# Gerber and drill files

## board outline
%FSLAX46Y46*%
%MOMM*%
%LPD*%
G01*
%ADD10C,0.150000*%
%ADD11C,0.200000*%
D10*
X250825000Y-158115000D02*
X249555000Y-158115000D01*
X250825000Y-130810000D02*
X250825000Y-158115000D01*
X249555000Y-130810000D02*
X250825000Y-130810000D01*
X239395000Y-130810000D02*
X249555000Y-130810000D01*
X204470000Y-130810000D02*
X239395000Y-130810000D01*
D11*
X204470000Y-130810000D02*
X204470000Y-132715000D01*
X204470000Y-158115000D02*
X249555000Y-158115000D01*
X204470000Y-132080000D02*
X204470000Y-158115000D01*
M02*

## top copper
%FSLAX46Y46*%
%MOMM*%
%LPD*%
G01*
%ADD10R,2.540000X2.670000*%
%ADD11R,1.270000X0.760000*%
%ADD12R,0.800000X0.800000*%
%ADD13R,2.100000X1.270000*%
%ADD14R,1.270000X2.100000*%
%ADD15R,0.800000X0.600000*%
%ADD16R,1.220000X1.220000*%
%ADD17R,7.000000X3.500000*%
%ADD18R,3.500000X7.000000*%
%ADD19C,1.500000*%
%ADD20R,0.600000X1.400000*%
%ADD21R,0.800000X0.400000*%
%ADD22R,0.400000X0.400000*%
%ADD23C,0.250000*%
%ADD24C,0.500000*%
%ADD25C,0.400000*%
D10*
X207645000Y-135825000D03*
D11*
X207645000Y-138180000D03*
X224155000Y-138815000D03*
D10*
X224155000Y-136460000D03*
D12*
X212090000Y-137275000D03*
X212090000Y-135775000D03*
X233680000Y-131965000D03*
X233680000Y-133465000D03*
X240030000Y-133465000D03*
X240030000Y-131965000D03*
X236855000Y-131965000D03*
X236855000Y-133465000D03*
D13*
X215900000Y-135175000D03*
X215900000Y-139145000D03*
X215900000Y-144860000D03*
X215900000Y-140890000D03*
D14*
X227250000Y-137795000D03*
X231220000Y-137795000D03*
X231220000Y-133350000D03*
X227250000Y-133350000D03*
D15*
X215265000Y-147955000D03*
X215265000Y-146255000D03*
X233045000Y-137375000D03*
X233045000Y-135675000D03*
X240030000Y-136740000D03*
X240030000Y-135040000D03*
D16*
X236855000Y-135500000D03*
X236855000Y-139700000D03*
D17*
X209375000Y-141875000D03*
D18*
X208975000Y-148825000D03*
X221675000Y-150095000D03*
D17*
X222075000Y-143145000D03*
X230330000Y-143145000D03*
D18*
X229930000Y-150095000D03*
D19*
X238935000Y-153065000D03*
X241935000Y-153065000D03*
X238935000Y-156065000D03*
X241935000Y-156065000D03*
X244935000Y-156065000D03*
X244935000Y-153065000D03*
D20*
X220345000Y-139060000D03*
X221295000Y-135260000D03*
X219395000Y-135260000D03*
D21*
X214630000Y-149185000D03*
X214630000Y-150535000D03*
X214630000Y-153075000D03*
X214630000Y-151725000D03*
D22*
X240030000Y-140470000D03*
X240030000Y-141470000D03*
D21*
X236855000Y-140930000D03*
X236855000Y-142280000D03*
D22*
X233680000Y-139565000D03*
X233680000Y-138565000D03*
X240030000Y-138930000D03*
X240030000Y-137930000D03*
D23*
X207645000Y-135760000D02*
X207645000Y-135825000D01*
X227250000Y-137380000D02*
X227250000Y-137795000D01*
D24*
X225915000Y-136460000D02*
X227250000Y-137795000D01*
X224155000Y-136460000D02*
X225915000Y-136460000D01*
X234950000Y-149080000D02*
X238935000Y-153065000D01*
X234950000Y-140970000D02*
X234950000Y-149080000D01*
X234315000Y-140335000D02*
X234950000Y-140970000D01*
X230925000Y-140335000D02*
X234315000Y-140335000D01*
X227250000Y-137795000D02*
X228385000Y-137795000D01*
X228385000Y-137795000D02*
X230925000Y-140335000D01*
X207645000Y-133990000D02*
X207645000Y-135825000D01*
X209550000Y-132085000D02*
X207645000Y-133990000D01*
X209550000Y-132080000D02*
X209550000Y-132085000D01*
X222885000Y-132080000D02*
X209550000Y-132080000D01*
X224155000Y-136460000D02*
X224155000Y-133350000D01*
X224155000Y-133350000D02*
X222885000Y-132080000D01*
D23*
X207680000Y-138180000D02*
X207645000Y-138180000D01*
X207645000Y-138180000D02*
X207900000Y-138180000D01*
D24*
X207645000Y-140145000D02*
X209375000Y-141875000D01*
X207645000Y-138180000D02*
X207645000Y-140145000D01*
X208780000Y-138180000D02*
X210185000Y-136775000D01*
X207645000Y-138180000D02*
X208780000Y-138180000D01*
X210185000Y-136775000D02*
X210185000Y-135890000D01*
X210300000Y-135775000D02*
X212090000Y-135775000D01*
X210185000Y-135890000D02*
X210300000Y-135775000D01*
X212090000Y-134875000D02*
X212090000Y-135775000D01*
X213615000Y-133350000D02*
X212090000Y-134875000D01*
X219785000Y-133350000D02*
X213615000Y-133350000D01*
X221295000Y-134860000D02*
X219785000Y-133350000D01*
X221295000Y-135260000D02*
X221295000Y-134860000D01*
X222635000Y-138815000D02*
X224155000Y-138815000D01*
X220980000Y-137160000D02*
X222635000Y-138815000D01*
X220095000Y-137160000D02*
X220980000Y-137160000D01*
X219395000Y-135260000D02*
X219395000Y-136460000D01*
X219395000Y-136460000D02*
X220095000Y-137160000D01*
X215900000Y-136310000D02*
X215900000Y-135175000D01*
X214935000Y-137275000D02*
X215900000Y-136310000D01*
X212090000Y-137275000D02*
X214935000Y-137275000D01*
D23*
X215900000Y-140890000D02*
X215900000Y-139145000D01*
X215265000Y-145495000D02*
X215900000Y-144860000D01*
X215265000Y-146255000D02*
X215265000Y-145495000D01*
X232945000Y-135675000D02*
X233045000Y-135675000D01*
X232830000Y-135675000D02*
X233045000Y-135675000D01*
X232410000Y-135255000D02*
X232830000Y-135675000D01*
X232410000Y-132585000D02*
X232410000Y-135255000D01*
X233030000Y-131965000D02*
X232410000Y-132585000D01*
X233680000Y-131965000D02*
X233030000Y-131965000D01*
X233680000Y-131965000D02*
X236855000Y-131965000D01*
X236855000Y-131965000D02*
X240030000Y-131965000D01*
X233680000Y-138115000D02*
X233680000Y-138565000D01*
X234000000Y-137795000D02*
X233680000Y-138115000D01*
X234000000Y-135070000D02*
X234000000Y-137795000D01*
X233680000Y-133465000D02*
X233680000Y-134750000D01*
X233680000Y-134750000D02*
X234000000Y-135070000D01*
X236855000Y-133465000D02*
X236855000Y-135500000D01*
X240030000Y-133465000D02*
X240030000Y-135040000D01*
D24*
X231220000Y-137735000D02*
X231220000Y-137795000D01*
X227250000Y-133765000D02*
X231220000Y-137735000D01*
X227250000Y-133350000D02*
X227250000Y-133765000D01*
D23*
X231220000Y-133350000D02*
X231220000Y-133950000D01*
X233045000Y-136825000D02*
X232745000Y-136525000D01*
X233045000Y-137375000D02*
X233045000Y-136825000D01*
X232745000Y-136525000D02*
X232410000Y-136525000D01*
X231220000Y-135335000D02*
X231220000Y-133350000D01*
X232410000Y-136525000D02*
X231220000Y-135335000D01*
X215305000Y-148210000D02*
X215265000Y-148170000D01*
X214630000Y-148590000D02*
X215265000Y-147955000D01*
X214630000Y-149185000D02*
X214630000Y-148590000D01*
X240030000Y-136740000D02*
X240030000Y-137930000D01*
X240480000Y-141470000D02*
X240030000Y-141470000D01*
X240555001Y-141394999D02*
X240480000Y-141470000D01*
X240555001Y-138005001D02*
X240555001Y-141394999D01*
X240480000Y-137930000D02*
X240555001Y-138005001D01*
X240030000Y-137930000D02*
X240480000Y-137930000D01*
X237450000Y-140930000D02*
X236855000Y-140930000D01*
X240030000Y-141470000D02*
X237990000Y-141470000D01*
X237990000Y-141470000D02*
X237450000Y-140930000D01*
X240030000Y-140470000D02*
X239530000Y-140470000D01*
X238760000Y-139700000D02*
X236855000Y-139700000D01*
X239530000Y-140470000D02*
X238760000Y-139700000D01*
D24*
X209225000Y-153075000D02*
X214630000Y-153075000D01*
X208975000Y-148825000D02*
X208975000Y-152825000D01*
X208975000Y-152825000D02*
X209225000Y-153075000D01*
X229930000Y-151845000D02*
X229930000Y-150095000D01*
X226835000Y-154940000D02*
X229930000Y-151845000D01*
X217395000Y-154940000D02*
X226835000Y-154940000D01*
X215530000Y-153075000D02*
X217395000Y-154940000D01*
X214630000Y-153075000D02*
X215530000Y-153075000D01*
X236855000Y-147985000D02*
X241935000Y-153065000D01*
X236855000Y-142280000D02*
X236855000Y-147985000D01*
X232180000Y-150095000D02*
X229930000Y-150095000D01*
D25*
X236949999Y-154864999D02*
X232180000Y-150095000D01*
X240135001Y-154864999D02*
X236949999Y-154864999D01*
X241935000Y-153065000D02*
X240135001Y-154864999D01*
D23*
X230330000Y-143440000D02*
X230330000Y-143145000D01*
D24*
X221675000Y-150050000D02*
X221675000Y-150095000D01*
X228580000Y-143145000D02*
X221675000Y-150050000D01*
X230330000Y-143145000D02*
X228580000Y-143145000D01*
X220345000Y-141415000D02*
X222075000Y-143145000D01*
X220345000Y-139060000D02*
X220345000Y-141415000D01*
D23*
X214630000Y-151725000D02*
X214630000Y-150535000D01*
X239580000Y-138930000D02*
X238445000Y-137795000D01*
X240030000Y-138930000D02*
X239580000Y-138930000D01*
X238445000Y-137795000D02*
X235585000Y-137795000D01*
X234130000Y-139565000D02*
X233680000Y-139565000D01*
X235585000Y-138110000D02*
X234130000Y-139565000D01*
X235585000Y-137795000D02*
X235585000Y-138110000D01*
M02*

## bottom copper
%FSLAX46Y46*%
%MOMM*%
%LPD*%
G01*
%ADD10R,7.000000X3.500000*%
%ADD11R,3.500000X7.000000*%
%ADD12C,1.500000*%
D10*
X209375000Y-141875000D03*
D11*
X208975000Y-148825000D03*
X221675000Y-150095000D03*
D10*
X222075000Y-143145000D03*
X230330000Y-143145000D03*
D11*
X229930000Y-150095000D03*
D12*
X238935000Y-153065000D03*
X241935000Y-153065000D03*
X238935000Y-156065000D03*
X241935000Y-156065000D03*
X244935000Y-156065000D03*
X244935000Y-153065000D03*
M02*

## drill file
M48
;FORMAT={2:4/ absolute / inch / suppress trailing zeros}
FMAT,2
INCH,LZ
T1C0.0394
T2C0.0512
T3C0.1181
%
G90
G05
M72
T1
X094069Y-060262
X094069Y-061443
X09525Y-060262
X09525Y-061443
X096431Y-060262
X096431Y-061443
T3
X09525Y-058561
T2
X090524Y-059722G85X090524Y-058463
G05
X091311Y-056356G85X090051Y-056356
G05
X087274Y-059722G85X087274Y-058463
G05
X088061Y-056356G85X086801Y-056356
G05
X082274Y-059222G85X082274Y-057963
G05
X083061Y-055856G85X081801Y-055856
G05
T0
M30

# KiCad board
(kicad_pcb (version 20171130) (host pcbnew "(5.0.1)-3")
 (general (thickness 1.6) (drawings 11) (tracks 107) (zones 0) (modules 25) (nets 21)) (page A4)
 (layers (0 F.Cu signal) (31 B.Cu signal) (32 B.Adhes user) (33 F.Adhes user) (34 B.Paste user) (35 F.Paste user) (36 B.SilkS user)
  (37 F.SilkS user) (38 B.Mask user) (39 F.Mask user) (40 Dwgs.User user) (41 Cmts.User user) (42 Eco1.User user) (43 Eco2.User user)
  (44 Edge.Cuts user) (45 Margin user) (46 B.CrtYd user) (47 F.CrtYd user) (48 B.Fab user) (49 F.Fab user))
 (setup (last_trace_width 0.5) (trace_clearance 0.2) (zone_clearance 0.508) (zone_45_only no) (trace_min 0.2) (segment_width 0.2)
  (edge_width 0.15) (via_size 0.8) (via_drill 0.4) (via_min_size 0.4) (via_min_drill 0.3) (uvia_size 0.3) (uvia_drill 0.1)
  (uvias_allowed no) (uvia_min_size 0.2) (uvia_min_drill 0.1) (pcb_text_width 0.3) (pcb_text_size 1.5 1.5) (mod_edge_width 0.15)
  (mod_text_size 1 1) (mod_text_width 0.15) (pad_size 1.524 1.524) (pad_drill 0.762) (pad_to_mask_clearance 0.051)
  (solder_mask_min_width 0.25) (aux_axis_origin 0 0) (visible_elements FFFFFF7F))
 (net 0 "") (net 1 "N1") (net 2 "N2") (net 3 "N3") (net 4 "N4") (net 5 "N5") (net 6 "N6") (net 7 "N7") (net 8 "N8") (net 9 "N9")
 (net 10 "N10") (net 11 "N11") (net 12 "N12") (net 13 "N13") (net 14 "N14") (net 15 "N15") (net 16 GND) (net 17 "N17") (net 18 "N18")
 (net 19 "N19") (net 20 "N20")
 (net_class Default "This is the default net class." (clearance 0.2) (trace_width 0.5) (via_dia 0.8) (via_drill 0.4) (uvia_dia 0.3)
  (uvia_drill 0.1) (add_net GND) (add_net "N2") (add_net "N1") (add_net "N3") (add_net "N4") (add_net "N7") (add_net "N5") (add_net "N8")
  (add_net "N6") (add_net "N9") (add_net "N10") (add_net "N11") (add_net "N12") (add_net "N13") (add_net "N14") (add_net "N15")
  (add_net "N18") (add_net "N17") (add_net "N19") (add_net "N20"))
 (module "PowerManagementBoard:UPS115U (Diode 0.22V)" (layer F.Cu) (at 207.645 137.16 270)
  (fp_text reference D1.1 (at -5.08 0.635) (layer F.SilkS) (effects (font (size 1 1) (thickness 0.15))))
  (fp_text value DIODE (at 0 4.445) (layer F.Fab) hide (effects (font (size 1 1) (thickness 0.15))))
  (pad 2 smd rect (at -1.335 0 270) (size 2.67 2.54) (layers F.Cu F.Paste F.Mask) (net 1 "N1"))
  (pad 1 smd rect (at 1.02 0 270) (size 0.76 1.27) (layers F.Cu F.Paste F.Mask) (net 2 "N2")))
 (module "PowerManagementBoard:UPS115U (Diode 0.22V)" (layer F.Cu) (at 224.155 137.795 270)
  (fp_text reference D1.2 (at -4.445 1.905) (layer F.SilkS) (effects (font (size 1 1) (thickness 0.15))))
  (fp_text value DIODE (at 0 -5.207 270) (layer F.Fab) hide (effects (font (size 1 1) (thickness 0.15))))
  (pad 1 smd rect (at 1.02 0 270) (size 0.76 1.27) (layers F.Cu F.Paste F.Mask) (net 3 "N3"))
  (pad 2 smd rect (at -1.335 0 270) (size 2.67 2.54) (layers F.Cu F.Paste F.Mask) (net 1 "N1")))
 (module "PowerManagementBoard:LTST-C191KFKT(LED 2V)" (layer F.Cu) (at 212.09 136.525 90)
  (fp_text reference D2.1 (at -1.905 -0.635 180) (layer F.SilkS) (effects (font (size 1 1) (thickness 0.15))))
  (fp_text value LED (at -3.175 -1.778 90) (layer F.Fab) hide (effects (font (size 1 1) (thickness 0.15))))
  (pad 1 smd rect (at -0.75 0 90) (size 0.8 0.8) (layers F.Cu B.Adhes F.Paste F.Mask) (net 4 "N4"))
  (pad 2 smd rect (at 0.75 0 90) (size 0.8 0.8) (layers F.Cu F.Paste F.Mask) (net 2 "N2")))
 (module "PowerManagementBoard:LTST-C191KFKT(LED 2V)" (layer F.Cu) (at 233.68 132.715 90)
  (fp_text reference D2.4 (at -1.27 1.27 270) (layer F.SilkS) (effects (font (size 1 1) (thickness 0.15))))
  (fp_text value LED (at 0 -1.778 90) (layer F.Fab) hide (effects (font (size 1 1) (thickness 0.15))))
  (pad 2 smd rect (at 0.75 0 90) (size 0.8 0.8) (layers F.Cu F.Paste F.Mask) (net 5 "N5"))
  (pad 1 smd rect (at -0.75 0 90) (size 0.8 0.8) (layers F.Cu B.Adhes F.Paste F.Mask) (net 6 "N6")))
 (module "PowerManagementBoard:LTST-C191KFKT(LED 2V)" (layer F.Cu) (at 240.03 132.715 90)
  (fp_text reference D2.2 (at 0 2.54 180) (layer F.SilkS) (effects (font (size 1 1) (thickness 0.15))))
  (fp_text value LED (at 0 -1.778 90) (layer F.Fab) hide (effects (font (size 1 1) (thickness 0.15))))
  (pad 1 smd rect (at -0.75 0 90) (size 0.8 0.8) (layers F.Cu B.Adhes F.Paste F.Mask) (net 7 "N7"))
  (pad 2 smd rect (at 0.75 0 90) (size 0.8 0.8) (layers F.Cu F.Paste F.Mask) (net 5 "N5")))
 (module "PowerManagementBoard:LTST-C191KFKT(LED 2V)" (layer F.Cu) (at 236.855 132.715 90)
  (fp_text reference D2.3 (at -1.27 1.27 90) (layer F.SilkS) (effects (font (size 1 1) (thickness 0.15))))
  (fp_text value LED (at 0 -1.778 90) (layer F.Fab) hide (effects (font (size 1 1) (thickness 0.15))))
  (pad 2 smd rect (at 0.75 0 90) (size 0.8 0.8) (layers F.Cu F.Paste F.Mask) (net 5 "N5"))
  (pad 1 smd rect (at -0.75 0 90) (size 0.8 0.8) (layers F.Cu B.Adhes F.Paste F.Mask) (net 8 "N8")))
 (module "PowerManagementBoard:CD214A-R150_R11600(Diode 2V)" (layer F.Cu) (at 215.9 137.16 270)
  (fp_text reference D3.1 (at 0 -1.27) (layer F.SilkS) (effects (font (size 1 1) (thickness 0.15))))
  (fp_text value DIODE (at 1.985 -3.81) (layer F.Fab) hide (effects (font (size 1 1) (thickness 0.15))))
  (pad 1 smd rect (at -1.985 0 270) (size 1.27 2.1) (layers F.Cu B.Adhes F.Paste F.Mask) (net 4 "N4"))
  (pad 2 smd rect (at 1.985 0 270) (size 1.27 2.1) (layers F.Cu B.Adhes F.Paste F.Mask) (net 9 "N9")))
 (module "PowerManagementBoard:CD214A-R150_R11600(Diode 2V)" (layer F.Cu) (at 215.9 142.875 270)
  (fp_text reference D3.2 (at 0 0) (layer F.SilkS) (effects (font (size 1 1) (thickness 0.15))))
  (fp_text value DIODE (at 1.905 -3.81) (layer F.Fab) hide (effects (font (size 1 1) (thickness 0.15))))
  (pad 2 smd rect (at 1.985 0 270) (size 1.27 2.1) (layers F.Cu B.Adhes F.Paste F.Mask) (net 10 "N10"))
  (pad 1 smd rect (at -1.985 0 270) (size 1.27 2.1) (layers F.Cu B.Adhes F.Paste F.Mask) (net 9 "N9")))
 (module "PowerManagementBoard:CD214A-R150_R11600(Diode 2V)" (layer F.Cu) (at 229.235 137.795)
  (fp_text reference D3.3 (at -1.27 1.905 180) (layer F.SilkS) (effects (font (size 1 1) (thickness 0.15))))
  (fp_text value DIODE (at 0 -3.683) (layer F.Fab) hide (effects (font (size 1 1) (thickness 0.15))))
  (pad 1 smd rect (at -1.985 0) (size 1.27 2.1) (layers F.Cu B.Adhes F.Paste F.Mask) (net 1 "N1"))
  (pad 2 smd rect (at 1.985 0) (size 1.27 2.1) (layers F.Cu B.Adhes F.Paste F.Mask) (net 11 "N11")))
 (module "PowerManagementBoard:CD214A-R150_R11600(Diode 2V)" (layer F.Cu) (at 229.235 133.35)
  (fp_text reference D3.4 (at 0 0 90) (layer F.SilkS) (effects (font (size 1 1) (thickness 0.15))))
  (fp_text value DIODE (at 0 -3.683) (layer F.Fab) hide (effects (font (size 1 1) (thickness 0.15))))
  (pad 2 smd rect (at 1.985 0) (size 1.27 2.1) (layers F.Cu B.Adhes F.Paste F.Mask) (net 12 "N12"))
  (pad 1 smd rect (at -1.985 0) (size 1.27 2.1) (layers F.Cu B.Adhes F.Paste F.Mask) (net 11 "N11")))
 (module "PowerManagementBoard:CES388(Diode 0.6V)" (layer F.Cu) (at 215.265 147.105 270)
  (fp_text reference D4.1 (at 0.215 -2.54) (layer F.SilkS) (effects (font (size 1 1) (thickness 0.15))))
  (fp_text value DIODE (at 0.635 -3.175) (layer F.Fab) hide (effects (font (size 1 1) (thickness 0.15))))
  (pad 2 smd rect (at 0.85 0 270) (size 0.6 0.8) (layers F.Cu B.Adhes F.Paste F.Mask) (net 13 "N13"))
  (pad 1 smd rect (at -0.85 0 270) (size 0.6 0.8) (layers F.Cu B.Adhes F.Paste F.Mask) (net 10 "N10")))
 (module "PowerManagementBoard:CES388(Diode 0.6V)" (layer F.Cu) (at 233.045 136.525 90)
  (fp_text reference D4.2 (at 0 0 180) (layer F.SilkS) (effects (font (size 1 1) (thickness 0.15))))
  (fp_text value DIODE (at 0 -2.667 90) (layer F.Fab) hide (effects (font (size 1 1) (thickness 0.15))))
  (pad 1 smd rect (at -0.85 0 90) (size 0.6 0.8) (layers F.Cu B.Adhes F.Paste F.Mask) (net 12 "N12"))
  (pad 2 smd rect (at 0.85 0 90) (size 0.6 0.8) (layers F.Cu B.Adhes F.Paste F.Mask) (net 5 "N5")))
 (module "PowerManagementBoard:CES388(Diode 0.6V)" (layer F.Cu) (at 240.03 135.89 270)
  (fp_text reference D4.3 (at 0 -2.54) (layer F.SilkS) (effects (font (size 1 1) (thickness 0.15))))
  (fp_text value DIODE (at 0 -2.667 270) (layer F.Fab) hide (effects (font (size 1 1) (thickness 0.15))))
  (pad 2 smd rect (at 0.85 0 270) (size 0.6 0.8) (layers F.Cu B.Adhes F.Paste F.Mask) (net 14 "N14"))
  (pad 1 smd rect (at -0.85 0 270) (size 0.6 0.8) (layers F.Cu B.Adhes F.Paste F.Mask) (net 7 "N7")))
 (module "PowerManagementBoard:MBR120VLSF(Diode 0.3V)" (layer F.Cu) (at 236.855 137.6 90)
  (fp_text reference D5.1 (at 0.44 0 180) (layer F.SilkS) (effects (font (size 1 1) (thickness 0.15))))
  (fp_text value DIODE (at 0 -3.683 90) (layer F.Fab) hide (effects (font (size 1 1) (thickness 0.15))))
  (pad 1 smd rect (at 2.1 0 90) (size 1.22 1.22) (layers F.Cu B.Adhes F.Paste F.Mask) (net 8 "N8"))
  (pad 2 smd rect (at -2.1 0 90) (size 1.22 1.22) (layers F.Cu B.Adhes F.Paste F.Mask) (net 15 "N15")))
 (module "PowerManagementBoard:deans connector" (layer F.Cu) (at 206.375 142.875 180)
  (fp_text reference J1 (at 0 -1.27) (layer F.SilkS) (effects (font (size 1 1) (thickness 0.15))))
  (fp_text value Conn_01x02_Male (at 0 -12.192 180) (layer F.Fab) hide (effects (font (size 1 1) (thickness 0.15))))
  (pad 1 thru_hole rect (at -3 1 180) (size 7 3.5) (drill oval 4.5 1.3) (layers *.Cu *.Mask) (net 2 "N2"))
  (pad 2 thru_hole rect (at -2.6 -5.95 180) (size 3.5 7) (drill oval 1.3 4.5) (layers *.Cu *.Mask) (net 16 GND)))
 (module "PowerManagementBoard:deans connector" (layer F.Cu) (at 219.075 144.145 180)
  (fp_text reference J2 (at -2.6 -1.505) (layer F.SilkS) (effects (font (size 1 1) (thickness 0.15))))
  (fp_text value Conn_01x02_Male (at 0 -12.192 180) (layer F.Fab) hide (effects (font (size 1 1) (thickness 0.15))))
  (pad 2 thru_hole rect (at -2.6 -5.95 180) (size 3.5 7) (drill oval 1.3 4.5) (layers *.Cu *.Mask) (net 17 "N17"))
  (pad 1 thru_hole rect (at -3 1 180) (size 7 3.5) (drill oval 4.5 1.3) (layers *.Cu *.Mask) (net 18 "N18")))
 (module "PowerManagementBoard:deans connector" (layer F.Cu) (at 227.33 144.145 180)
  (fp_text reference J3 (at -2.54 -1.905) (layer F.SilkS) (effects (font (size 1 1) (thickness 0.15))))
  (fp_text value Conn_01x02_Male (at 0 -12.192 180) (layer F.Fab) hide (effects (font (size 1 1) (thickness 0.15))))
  (pad 1 thru_hole rect (at -3 1 180) (size 7 3.5) (drill oval 4.5 1.3) (layers *.Cu *.Mask) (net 17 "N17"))
  (pad 2 thru_hole rect (at -2.6 -5.95 180) (size 3.5 7) (drill oval 1.3 4.5) (layers *.Cu *.Mask) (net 16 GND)))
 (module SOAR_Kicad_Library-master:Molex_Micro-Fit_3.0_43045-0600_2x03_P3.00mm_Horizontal (layer F.Cu) (at 241.935 144.145 180)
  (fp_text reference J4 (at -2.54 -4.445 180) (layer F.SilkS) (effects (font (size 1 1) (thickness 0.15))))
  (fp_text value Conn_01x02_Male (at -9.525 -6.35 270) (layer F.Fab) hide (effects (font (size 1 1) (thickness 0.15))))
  (pad "" np_thru_hole circle (at 0 -4.6) (size 3 3) (drill 3) (layers *.Cu *.Mask))
  (pad 1 thru_hole circle (at 3 -8.92) (size 1.5 1.5) (drill 1) (layers *.Cu *.Mask) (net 1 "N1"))
  (pad 2 thru_hole circle (at 0 -8.92) (size 1.5 1.5) (drill 1) (layers *.Cu *.Mask) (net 16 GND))
  (pad 4 thru_hole circle (at 3 -11.92) (size 1.5 1.5) (drill 1) (layers *.Cu *.Mask))
  (pad 5 thru_hole circle (at 0 -11.92) (size 1.5 1.5) (drill 1) (layers *.Cu *.Mask))
  (pad 6 thru_hole circle (at -3 -11.92) (size 1.5 1.5) (drill 1) (layers *.Cu *.Mask))
  (pad 3 thru_hole circle (at -3 -8.92) (size 1.5 1.5) (drill 1) (layers *.Cu *.Mask)))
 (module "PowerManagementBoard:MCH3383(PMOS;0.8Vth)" (layer F.Cu) (at 220.345 137.16 180)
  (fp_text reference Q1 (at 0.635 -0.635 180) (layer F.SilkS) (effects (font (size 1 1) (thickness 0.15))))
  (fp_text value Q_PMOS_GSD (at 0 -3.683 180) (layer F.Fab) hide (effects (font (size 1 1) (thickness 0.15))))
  (pad 3 smd rect (at 0 -1.9 180) (size 0.6 1.4) (layers F.Cu F.Paste F.Mask) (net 18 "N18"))
  (pad 1 smd rect (at -0.95 1.9 180) (size 0.6 1.4) (layers F.Cu F.Paste F.Mask) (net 2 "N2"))
  (pad 2 smd rect (at 0.95 1.9 180) (size 0.6 1.4) (layers F.Cu F.Paste F.Mask) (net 3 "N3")))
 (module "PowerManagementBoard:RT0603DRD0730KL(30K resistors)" (layer F.Cu) (at 214.63 149.86 90)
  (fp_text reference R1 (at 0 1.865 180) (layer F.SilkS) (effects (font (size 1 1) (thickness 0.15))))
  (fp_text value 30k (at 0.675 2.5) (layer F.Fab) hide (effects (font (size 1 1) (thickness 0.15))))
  (pad 1 smd rect (at 0.675 0 90) (size 0.4 0.8) (layers F.Cu B.Adhes F.Paste F.Mask) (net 13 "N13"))
  (pad 2 smd rect (at -0.675 0 90) (size 0.4 0.8) (layers F.Cu B.Adhes F.Paste F.Mask) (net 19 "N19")))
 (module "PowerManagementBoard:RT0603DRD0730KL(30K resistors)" (layer F.Cu) (at 214.63 152.4 90)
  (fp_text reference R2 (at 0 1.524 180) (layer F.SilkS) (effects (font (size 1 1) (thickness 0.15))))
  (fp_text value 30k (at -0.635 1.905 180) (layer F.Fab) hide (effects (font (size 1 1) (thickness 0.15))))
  (pad 2 smd rect (at -0.675 0 90) (size 0.4 0.8) (layers F.Cu B.Adhes F.Paste F.Mask) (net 16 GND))
  (pad 1 smd rect (at 0.675 0 90) (size 0.4 0.8) (layers F.Cu B.Adhes F.Paste F.Mask) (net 19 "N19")))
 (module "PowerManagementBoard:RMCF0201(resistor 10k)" (layer F.Cu) (at 240.03 140.97 90)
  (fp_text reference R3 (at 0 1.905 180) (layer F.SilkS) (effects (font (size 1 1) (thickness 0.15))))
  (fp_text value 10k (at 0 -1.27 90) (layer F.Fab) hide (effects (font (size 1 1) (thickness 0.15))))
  (pad 1 smd rect (at 0.5 0 90) (size 0.4 0.4) (layers F.Cu B.Adhes F.Paste F.Mask) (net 15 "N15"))
  (pad 2 smd rect (at -0.5 0 90) (size 0.4 0.4) (layers F.Cu B.Adhes F.Paste F.Mask) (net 14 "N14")))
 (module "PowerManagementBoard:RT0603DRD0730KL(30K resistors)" (layer F.Cu) (at 236.855 141.605 90)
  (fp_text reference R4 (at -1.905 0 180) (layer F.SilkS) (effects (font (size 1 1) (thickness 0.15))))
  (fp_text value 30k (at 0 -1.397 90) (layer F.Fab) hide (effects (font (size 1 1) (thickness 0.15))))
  (pad 1 smd rect (at 0.675 0 90) (size 0.4 0.8) (layers F.Cu B.Adhes F.Paste F.Mask) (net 14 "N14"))
  (pad 2 smd rect (at -0.675 0 90) (size 0.4 0.8) (layers F.Cu B.Adhes F.Paste F.Mask) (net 16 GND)))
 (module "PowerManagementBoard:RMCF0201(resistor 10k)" (layer F.Cu) (at 233.68 139.065 90)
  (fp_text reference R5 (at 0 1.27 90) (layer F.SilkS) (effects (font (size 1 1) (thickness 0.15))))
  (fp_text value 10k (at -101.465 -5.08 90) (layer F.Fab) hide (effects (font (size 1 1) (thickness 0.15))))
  (pad 2 smd rect (at -0.5 0 90) (size 0.4 0.4) (layers F.Cu B.Adhes F.Paste F.Mask) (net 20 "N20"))
  (pad 1 smd rect (at 0.5 0 90) (size 0.4 0.4) (layers F.Cu B.Adhes F.Paste F.Mask) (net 6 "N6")))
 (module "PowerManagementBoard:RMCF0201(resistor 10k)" (layer F.Cu) (at 240.03 138.43 270)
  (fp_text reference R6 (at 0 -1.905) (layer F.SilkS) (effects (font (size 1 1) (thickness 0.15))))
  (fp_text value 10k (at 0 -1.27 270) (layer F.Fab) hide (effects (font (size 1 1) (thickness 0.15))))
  (pad 1 smd rect (at 0.5 0 270) (size 0.4 0.4) (layers F.Cu B.Adhes F.Paste F.Mask) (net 20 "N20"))
  (pad 2 smd rect (at -0.5 0 270) (size 0.4 0.4) (layers F.Cu B.Adhes F.Paste F.Mask) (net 14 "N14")))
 (gr_line (start 250.825 158.115) (end 249.555 158.115) (layer Edge.Cuts) (width 0.15))
 (gr_line (start 250.825 130.81) (end 250.825 158.115) (layer Edge.Cuts) (width 0.15))
 (gr_line (start 249.555 130.81) (end 250.825 130.81) (layer Edge.Cuts) (width 0.15))
 (gr_line (start 239.395 130.81) (end 249.555 130.81) (layer Edge.Cuts) (width 0.15))
 (gr_line (start 204.47 130.81) (end 239.395 130.81) (layer Edge.Cuts) (width 0.15))
 (gr_line (start 204.47 130.81) (end 204.47 132.715) (layer Edge.Cuts) (width 0.2))
 (gr_line (start 204.47 158.115) (end 249.555 158.115) (layer Edge.Cuts) (width 0.2))
 (gr_line (start 204.47 132.08) (end 204.47 158.115) (layer Edge.Cuts) (width 0.2))
 (segment (start 207.645 135.76) (end 207.645 135.825) (width 0.25) (layer F.Cu) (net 1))
 (segment (start 227.25 137.38) (end 227.25 137.795) (width 0.25) (layer F.Cu) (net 1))
 (segment (start 225.915 136.46) (end 227.25 137.795) (width 0.5) (layer F.Cu) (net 1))
 (segment (start 224.155 136.46) (end 225.915 136.46) (width 0.5) (layer F.Cu) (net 1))
 (segment (start 234.95 149.08) (end 238.935 153.065) (width 0.5) (layer F.Cu) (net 1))
 (segment (start 234.95 140.97) (end 234.95 149.08) (width 0.5) (layer F.Cu) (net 1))
 (segment (start 234.315 140.335) (end 234.95 140.97) (width 0.5) (layer F.Cu) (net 1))
 (segment (start 230.925 140.335) (end 234.315 140.335) (width 0.5) (layer F.Cu) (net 1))
 (segment (start 227.25 137.795) (end 228.385 137.795) (width 0.5) (layer F.Cu) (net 1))
 (segment (start 228.385 137.795) (end 230.925 140.335) (width 0.5) (layer F.Cu) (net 1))
 (segment (start 207.645 133.99) (end 207.645 135.825) (width 0.5) (layer F.Cu) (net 1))
 (segment (start 209.55 132.085) (end 207.645 133.99) (width 0.5) (layer F.Cu) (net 1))
 (segment (start 209.55 132.08) (end 209.55 132.085) (width 0.5) (layer F.Cu) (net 1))
 (segment (start 222.885 132.08) (end 209.55 132.08) (width 0.5) (layer F.Cu) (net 1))
 (segment (start 224.155 136.46) (end 224.155 133.35) (width 0.5) (layer F.Cu) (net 1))
 (segment (start 224.155 133.35) (end 222.885 132.08) (width 0.5) (layer F.Cu) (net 1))
 (segment (start 207.68 138.18) (end 207.645 138.18) (width 0.25) (layer F.Cu) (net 2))
 (segment (start 207.645 138.18) (end 207.9 138.18) (width 0.25) (layer F.Cu) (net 2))
 (segment (start 207.645 140.145) (end 209.375 141.875) (width 0.5) (layer F.Cu) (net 2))
 (segment (start 207.645 138.18) (end 207.645 140.145) (width 0.5) (layer F.Cu) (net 2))
 (segment (start 208.78 138.18) (end 210.185 136.775) (width 0.5) (layer F.Cu) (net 2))
 (segment (start 207.645 138.18) (end 208.78 138.18) (width 0.5) (layer F.Cu) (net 2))
 (segment (start 210.185 136.775) (end 210.185 135.89) (width 0.5) (layer F.Cu) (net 2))
 (segment (start 210.3 135.775) (end 212.09 135.775) (width 0.5) (layer F.Cu) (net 2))
 (segment (start 210.185 135.89) (end 210.3 135.775) (width 0.5) (layer F.Cu) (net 2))
 (segment (start 212.09 134.875) (end 212.09 135.775) (width 0.5) (layer F.Cu) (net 2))
 (segment (start 213.615 133.35) (end 212.09 134.875) (width 0.5) (layer F.Cu) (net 2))
 (segment (start 219.785 133.35) (end 213.615 133.35) (width 0.5) (layer F.Cu) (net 2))
 (segment (start 221.295 134.86) (end 219.785 133.35) (width 0.5) (layer F.Cu) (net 2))
 (segment (start 221.295 135.26) (end 221.295 134.86) (width 0.5) (layer F.Cu) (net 2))
 (segment (start 222.635 138.815) (end 224.155 138.815) (width 0.5) (layer F.Cu) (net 3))
 (segment (start 220.98 137.16) (end 222.635 138.815) (width 0.5) (layer F.Cu) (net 3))
 (segment (start 220.095 137.16) (end 220.98 137.16) (width 0.5) (layer F.Cu) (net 3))
 (segment (start 219.395 135.26) (end 219.395 136.46) (width 0.5) (layer F.Cu) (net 3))
 (segment (start 219.395 136.46) (end 220.095 137.16) (width 0.5) (layer F.Cu) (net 3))
 (segment (start 215.9 136.31) (end 215.9 135.175) (width 0.5) (layer F.Cu) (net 4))
 (segment (start 214.935 137.275) (end 215.9 136.31) (width 0.5) (layer F.Cu) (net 4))
 (segment (start 212.09 137.275) (end 214.935 137.275) (width 0.5) (layer F.Cu) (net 4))
 (segment (start 215.9 140.89) (end 215.9 139.145) (width 0.25) (layer F.Cu) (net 9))
 (segment (start 215.265 145.495) (end 215.9 144.86) (width 0.25) (layer F.Cu) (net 10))
 (segment (start 215.265 146.255) (end 215.265 145.495) (width 0.25) (layer F.Cu) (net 10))
 (segment (start 232.945 135.675) (end 233.045 135.675) (width 0.25) (layer F.Cu) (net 5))
 (segment (start 232.83 135.675) (end 233.045 135.675) (width 0.25) (layer F.Cu) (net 5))
 (segment (start 232.41 135.255) (end 232.83 135.675) (width 0.25) (layer F.Cu) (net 5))
 (segment (start 232.41 132.585) (end 232.41 135.255) (width 0.25) (layer F.Cu) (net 5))
 (segment (start 233.03 131.965) (end 232.41 132.585) (width 0.25) (layer F.Cu) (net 5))
 (segment (start 233.68 131.965) (end 233.03 131.965) (width 0.25) (layer F.Cu) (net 5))
 (segment (start 233.68 131.965) (end 236.855 131.965) (width 0.25) (layer F.Cu) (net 5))
 (segment (start 236.855 131.965) (end 240.03 131.965) (width 0.25) (layer F.Cu) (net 5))
 (segment (start 233.68 138.115) (end 233.68 138.565) (width 0.25) (layer F.Cu) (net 6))
 (segment (start 234 137.795) (end 233.68 138.115) (width 0.25) (layer F.Cu) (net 6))
 (segment (start 234 135.07) (end 234 137.795) (width 0.25) (layer F.Cu) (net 6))
 (segment (start 233.68 133.465) (end 233.68 134.75) (width 0.25) (layer F.Cu) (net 6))
 (segment (start 233.68 134.75) (end 234 135.07) (width 0.25) (layer F.Cu) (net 6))
 (segment (start 236.855 133.465) (end 236.855 135.5) (width 0.25) (layer F.Cu) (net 8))
 (segment (start 240.03 133.465) (end 240.03 135.04) (width 0.25) (layer F.Cu) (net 7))
 (segment (start 231.22 137.735) (end 231.22 137.795) (width 0.5) (layer F.Cu) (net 11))
 (segment (start 227.25 133.765) (end 231.22 137.735) (width 0.5) (layer F.Cu) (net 11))
 (segment (start 227.25 133.35) (end 227.25 133.765) (width 0.5) (layer F.Cu) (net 11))
 (segment (start 231.22 133.35) (end 231.22 133.95) (width 0.25) (layer F.Cu) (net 12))
 (segment (start 233.045 136.825) (end 232.745 136.525) (width 0.25) (layer F.Cu) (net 12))
 (segment (start 233.045 137.375) (end 233.045 136.825) (width 0.25) (layer F.Cu) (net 12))
 (segment (start 232.745 136.525) (end 232.41 136.525) (width 0.25) (layer F.Cu) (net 12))
 (segment (start 231.22 135.335) (end 231.22 133.35) (width 0.25) (layer F.Cu) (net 12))
 (segment (start 232.41 136.525) (end 231.22 135.335) (width 0.25) (layer F.Cu) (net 12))
 (segment (start 215.305 148.21) (end 215.265 148.17) (width 0.25) (layer F.Cu) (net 13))
 (segment (start 214.63 148.59) (end 215.265 147.955) (width 0.25) (layer F.Cu) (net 13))
 (segment (start 214.63 149.185) (end 214.63 148.59) (width 0.25) (layer F.Cu) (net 13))
 (segment (start 240.03 136.74) (end 240.03 137.93) (width 0.25) (layer F.Cu) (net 14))
 (segment (start 240.48 141.47) (end 240.03 141.47) (width 0.25) (layer F.Cu) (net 14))
 (segment (start 240.555001 141.394999) (end 240.48 141.47) (width 0.25) (layer F.Cu) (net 14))
 (segment (start 240.555001 138.005001) (end 240.555001 141.394999) (width 0.25) (layer F.Cu) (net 14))
 (segment (start 240.48 137.93) (end 240.555001 138.005001) (width 0.25) (layer F.Cu) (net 14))
 (segment (start 240.03 137.93) (end 240.48 137.93) (width 0.25) (layer F.Cu) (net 14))
 (segment (start 237.45 140.93) (end 236.855 140.93) (width 0.25) (layer F.Cu) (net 14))
 (segment (start 240.03 141.47) (end 237.99 141.47) (width 0.25) (layer F.Cu) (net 14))
 (segment (start 237.99 141.47) (end 237.45 140.93) (width 0.25) (layer F.Cu) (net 14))
 (segment (start 240.03 140.47) (end 239.53 140.47) (width 0.25) (layer F.Cu) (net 15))
 (segment (start 238.76 139.7) (end 236.855 139.7) (width 0.25) (layer F.Cu) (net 15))
 (segment (start 239.53 140.47) (end 238.76 139.7) (width 0.25) (layer F.Cu) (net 15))
 (segment (start 209.225 153.075) (end 214.63 153.075) (width 0.5) (layer F.Cu) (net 16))
 (segment (start 208.975 148.825) (end 208.975 152.825) (width 0.5) (layer F.Cu) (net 16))
 (segment (start 208.975 152.825) (end 209.225 153.075) (width 0.5) (layer F.Cu) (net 16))
 (segment (start 229.93 151.845) (end 229.93 150.095) (width 0.5) (layer F.Cu) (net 16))
 (segment (start 226.835 154.94) (end 229.93 151.845) (width 0.5) (layer F.Cu) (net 16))
 (segment (start 217.395 154.94) (end 226.835 154.94) (width 0.5) (layer F.Cu) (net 16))
 (segment (start 215.53 153.075) (end 217.395 154.94) (width 0.5) (layer F.Cu) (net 16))
 (segment (start 214.63 153.075) (end 215.53 153.075) (width 0.5) (layer F.Cu) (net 16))
 (segment (start 236.855 147.985) (end 241.935 153.065) (width 0.5) (layer F.Cu) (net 16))
 (segment (start 236.855 142.28) (end 236.855 147.985) (width 0.5) (layer F.Cu) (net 16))
 (segment (start 232.18 150.095) (end 229.93 150.095) (width 0.5) (layer F.Cu) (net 16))
 (segment (start 236.949999 154.864999) (end 232.18 150.095) (width 0.4) (layer F.Cu) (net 16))
 (segment (start 240.135001 154.864999) (end 236.949999 154.864999) (width 0.4) (layer F.Cu) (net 16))
 (segment (start 241.935 153.065) (end 240.135001 154.864999) (width 0.4) (layer F.Cu) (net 16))
 (segment (start 230.33 143.44) (end 230.33 143.145) (width 0.25) (layer F.Cu) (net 17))
 (segment (start 221.675 150.05) (end 221.675 150.095) (width 0.5) (layer F.Cu) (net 17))
 (segment (start 228.58 143.145) (end 221.675 150.05) (width 0.5) (layer F.Cu) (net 17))
 (segment (start 230.33 143.145) (end 228.58 143.145) (width 0.5) (layer F.Cu) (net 17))
 (segment (start 220.345 141.415) (end 222.075 143.145) (width 0.5) (layer F.Cu) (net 18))
 (segment (start 220.345 139.06) (end 220.345 141.415) (width 0.5) (layer F.Cu) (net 18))
 (segment (start 214.63 151.725) (end 214.63 150.535) (width 0.25) (layer F.Cu) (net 19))
 (segment (start 239.58 138.93) (end 238.445 137.795) (width 0.25) (layer F.Cu) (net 20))
 (segment (start 240.03 138.93) (end 239.58 138.93) (width 0.25) (layer F.Cu) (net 20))
 (segment (start 238.445 137.795) (end 235.585 137.795) (width 0.25) (layer F.Cu) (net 20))
 (segment (start 234.13 139.565) (end 233.68 139.565) (width 0.25) (layer F.Cu) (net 20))
 (segment (start 235.585 138.11) (end 234.13 139.565) (width 0.25) (layer F.Cu) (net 20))
 (segment (start 235.585 137.795) (end 235.585 138.11) (width 0.25) (layer F.Cu) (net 20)))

